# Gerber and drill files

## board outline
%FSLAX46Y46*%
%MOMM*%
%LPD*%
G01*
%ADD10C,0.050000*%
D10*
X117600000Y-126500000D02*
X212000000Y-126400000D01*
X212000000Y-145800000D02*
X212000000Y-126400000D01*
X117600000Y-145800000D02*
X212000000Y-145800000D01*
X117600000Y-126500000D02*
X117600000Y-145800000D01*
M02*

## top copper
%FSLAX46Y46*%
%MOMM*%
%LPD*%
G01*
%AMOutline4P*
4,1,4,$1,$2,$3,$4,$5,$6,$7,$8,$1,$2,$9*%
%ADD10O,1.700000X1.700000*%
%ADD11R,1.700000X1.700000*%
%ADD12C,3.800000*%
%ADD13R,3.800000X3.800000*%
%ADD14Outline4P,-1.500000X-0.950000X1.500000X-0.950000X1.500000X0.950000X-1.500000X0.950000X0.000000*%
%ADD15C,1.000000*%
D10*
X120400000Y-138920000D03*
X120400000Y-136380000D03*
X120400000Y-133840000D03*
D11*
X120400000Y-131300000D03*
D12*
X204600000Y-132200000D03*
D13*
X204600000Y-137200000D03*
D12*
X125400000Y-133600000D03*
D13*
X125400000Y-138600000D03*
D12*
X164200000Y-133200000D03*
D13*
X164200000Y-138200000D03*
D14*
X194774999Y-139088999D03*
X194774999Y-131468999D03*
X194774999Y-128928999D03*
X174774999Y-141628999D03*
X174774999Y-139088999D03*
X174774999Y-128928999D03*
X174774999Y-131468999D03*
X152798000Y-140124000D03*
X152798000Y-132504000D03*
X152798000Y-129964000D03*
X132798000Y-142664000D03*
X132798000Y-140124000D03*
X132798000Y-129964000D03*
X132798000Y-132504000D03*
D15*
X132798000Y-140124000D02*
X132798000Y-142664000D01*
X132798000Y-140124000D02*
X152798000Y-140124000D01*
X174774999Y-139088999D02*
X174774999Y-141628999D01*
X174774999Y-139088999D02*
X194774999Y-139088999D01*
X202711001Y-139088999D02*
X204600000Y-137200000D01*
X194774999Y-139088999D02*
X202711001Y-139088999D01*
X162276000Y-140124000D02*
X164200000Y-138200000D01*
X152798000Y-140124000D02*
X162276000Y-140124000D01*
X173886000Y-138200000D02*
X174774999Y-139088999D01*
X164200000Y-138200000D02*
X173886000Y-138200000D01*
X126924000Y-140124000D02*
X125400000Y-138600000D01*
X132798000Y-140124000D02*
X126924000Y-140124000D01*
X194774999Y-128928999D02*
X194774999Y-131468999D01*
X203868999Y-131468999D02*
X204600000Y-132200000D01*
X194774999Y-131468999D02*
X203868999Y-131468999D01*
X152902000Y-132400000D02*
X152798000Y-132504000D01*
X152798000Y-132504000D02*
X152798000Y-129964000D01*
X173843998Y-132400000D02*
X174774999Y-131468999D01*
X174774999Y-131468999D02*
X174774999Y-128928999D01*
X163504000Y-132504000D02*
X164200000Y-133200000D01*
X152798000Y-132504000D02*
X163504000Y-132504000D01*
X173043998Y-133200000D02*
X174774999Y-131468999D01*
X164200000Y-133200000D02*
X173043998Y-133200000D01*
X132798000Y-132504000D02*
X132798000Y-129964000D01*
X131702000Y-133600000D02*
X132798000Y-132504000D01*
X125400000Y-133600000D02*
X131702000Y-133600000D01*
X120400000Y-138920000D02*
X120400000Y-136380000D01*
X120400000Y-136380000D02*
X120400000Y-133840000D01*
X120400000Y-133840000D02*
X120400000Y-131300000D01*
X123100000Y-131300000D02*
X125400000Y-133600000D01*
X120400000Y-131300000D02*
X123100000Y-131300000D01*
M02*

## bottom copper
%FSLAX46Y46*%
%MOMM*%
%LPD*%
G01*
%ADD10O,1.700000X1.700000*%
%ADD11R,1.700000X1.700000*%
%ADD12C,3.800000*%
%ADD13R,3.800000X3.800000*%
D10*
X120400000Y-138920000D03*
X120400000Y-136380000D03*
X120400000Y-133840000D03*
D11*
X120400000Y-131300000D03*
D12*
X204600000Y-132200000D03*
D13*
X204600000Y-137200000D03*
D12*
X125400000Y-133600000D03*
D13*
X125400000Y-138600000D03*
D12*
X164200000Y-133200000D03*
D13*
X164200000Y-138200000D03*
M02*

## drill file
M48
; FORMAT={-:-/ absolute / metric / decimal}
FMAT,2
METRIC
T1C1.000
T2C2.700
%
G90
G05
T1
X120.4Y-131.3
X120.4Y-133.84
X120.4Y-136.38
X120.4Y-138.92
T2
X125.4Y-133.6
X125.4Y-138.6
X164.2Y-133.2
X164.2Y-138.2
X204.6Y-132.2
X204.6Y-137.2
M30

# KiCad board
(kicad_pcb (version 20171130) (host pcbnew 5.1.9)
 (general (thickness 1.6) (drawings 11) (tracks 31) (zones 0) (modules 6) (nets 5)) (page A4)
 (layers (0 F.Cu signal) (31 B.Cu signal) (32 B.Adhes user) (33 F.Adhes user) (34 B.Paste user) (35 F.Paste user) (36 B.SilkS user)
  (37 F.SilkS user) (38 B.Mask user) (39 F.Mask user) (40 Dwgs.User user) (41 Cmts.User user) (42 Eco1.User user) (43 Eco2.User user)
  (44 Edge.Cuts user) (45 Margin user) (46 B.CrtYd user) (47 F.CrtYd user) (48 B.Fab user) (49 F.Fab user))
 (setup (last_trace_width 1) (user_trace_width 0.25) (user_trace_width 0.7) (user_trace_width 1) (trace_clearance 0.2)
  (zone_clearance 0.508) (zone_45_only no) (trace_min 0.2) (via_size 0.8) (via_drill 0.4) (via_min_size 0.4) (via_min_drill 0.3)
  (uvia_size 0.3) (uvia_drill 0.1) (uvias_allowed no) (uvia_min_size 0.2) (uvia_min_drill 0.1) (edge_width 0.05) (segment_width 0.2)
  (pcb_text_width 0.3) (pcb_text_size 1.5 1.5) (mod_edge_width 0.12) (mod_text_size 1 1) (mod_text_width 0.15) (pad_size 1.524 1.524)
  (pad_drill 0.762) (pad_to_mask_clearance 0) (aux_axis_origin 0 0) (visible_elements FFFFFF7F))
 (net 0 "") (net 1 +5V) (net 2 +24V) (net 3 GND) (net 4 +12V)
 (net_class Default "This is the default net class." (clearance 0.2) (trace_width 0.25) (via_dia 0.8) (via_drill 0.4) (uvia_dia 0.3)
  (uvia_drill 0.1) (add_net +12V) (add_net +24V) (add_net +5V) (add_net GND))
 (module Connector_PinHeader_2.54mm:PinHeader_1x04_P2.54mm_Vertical (layer F.Cu) (at 120.4 131.3)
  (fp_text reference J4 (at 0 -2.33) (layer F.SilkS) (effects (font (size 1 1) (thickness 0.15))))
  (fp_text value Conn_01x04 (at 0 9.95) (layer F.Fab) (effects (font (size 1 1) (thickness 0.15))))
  (pad 4 thru_hole oval (at 0 7.62) (size 1.7 1.7) (drill 1) (layers *.Cu *.Mask) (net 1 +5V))
  (pad 3 thru_hole oval (at 0 5.08) (size 1.7 1.7) (drill 1) (layers *.Cu *.Mask) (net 1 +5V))
  (pad 2 thru_hole oval (at 0 2.54) (size 1.7 1.7) (drill 1) (layers *.Cu *.Mask) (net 1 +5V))
  (pad 1 thru_hole rect (at 0 0) (size 1.7 1.7) (drill 1) (layers *.Cu *.Mask) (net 1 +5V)))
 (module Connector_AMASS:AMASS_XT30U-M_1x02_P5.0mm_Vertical (layer F.Cu) (at 204.6 137.2 90)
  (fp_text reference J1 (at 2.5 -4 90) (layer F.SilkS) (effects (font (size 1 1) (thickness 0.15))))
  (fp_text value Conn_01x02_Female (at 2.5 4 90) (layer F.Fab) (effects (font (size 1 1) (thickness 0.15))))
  (pad 2 thru_hole circle (at 5 0 90) (size 3.8 3.8) (drill 2.7) (layers *.Cu *.Mask) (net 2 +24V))
  (pad 1 thru_hole rect (at 0 0 90) (size 3.8 3.8) (drill 2.7) (layers *.Cu *.Mask) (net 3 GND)))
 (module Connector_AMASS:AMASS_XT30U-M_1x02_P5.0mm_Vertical (layer F.Cu) (at 125.4 138.6 90)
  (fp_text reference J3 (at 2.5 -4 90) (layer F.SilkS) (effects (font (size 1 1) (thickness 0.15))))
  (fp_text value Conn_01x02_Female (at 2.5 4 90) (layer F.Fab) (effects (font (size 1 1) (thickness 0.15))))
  (pad 2 thru_hole circle (at 5 0 90) (size 3.8 3.8) (drill 2.7) (layers *.Cu *.Mask) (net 1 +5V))
  (pad 1 thru_hole rect (at 0 0 90) (size 3.8 3.8) (drill 2.7) (layers *.Cu *.Mask) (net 3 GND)))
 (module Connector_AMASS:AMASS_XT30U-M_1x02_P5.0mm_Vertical (layer F.Cu) (at 164.2 138.2 90)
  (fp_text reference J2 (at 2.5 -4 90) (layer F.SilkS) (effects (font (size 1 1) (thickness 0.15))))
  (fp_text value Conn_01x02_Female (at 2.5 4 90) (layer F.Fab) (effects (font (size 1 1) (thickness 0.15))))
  (pad 2 thru_hole circle (at 5 0 90) (size 3.8 3.8) (drill 2.7) (layers *.Cu *.Mask) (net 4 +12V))
  (pad 1 thru_hole rect (at 0 0 90) (size 3.8 3.8) (drill 2.7) (layers *.Cu *.Mask) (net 3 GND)))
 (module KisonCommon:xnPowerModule (layer F.Cu) (at 178.076999 124.864999)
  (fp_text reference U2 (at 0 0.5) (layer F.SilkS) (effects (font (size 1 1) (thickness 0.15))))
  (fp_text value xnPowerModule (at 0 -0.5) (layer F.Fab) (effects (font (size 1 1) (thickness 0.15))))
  (pad 4 smd trapezoid (at 16.698 14.224) (size 3 1.9) (layers F.Cu F.Paste F.Mask) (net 3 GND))
  (pad 3 smd trapezoid (at 16.698 6.604) (size 3 1.9) (layers F.Cu F.Paste F.Mask) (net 2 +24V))
  (pad 3 smd trapezoid (at 16.698 4.064) (size 3 1.9) (layers F.Cu F.Paste F.Mask) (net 2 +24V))
  (pad 2 smd trapezoid (at -3.302 16.764) (size 3 1.9) (layers F.Cu F.Paste F.Mask) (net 3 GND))
  (pad 2 smd trapezoid (at -3.302 14.224) (size 3 1.9) (layers F.Cu F.Paste F.Mask) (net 3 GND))
  (pad 1 smd trapezoid (at -3.302 4.064) (size 3 1.9) (layers F.Cu F.Paste F.Mask) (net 4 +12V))
  (pad 1 smd trapezoid (at -3.302 6.604) (size 3 1.9) (layers F.Cu F.Paste F.Mask) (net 4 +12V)))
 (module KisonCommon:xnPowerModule (layer F.Cu) (at 136.1 125.9)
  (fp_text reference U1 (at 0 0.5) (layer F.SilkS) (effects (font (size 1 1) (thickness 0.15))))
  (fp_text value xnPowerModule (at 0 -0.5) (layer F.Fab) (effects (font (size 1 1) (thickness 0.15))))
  (pad 4 smd trapezoid (at 16.698 14.224) (size 3 1.9) (layers F.Cu F.Paste F.Mask) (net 3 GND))
  (pad 3 smd trapezoid (at 16.698 6.604) (size 3 1.9) (layers F.Cu F.Paste F.Mask) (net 4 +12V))
  (pad 3 smd trapezoid (at 16.698 4.064) (size 3 1.9) (layers F.Cu F.Paste F.Mask) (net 4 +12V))
  (pad 2 smd trapezoid (at -3.302 16.764) (size 3 1.9) (layers F.Cu F.Paste F.Mask) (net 3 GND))
  (pad 2 smd trapezoid (at -3.302 14.224) (size 3 1.9) (layers F.Cu F.Paste F.Mask) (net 3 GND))
  (pad 1 smd trapezoid (at -3.302 4.064) (size 3 1.9) (layers F.Cu F.Paste F.Mask) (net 1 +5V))
  (pad 1 smd trapezoid (at -3.302 6.604) (size 3 1.9) (layers F.Cu F.Paste F.Mask) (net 1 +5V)))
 (gr_line (start 117.6 126.5) (end 212 126.4) (layer Edge.Cuts) (width 0.05))
 (gr_line (start 212 145.8) (end 212 126.4) (layer Edge.Cuts) (width 0.05))
 (gr_line (start 117.6 145.8) (end 212 145.8) (layer Edge.Cuts) (width 0.05))
 (gr_line (start 117.6 126.5) (end 117.6 145.8) (layer Edge.Cuts) (width 0.05))
 (segment (start 132.798 140.124) (end 132.798 142.664) (width 1) (layer F.Cu) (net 3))
 (segment (start 132.798 140.124) (end 152.798 140.124) (width 1) (layer F.Cu) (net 3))
 (segment (start 174.774999 139.088999) (end 174.774999 141.628999) (width 1) (layer F.Cu) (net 3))
 (segment (start 174.774999 139.088999) (end 194.774999 139.088999) (width 1) (layer F.Cu) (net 3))
 (segment (start 202.711001 139.088999) (end 204.6 137.2) (width 1) (layer F.Cu) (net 3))
 (segment (start 194.774999 139.088999) (end 202.711001 139.088999) (width 1) (layer F.Cu) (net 3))
 (segment (start 162.276 140.124) (end 164.2 138.2) (width 1) (layer F.Cu) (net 3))
 (segment (start 152.798 140.124) (end 162.276 140.124) (width 1) (layer F.Cu) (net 3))
 (segment (start 173.886 138.2) (end 174.774999 139.088999) (width 1) (layer F.Cu) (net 3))
 (segment (start 164.2 138.2) (end 173.886 138.2) (width 1) (layer F.Cu) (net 3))
 (segment (start 126.924 140.124) (end 125.4 138.6) (width 1) (layer F.Cu) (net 3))
 (segment (start 132.798 140.124) (end 126.924 140.124) (width 1) (layer F.Cu) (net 3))
 (segment (start 194.774999 128.928999) (end 194.774999 131.468999) (width 1) (layer F.Cu) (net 2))
 (segment (start 203.868999 131.468999) (end 204.6 132.2) (width 1) (layer F.Cu) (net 2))
 (segment (start 194.774999 131.468999) (end 203.868999 131.468999) (width 1) (layer F.Cu) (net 2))
 (segment (start 152.902 132.4) (end 152.798 132.504) (width 1) (layer F.Cu) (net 4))
 (segment (start 152.798 132.504) (end 152.798 129.964) (width 1) (layer F.Cu) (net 4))
 (segment (start 173.843998 132.4) (end 174.774999 131.468999) (width 1) (layer F.Cu) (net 4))
 (segment (start 174.774999 131.468999) (end 174.774999 128.928999) (width 1) (layer F.Cu) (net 4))
 (segment (start 163.504 132.504) (end 164.2 133.2) (width 1) (layer F.Cu) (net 4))
 (segment (start 152.798 132.504) (end 163.504 132.504) (width 1) (layer F.Cu) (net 4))
 (segment (start 173.043998 133.2) (end 174.774999 131.468999) (width 1) (layer F.Cu) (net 4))
 (segment (start 164.2 133.2) (end 173.043998 133.2) (width 1) (layer F.Cu) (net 4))
 (segment (start 132.798 132.504) (end 132.798 129.964) (width 1) (layer F.Cu) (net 1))
 (segment (start 131.702 133.6) (end 132.798 132.504) (width 1) (layer F.Cu) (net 1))
 (segment (start 125.4 133.6) (end 131.702 133.6) (width 1) (layer F.Cu) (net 1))
 (segment (start 120.4 138.92) (end 120.4 136.38) (width 1) (layer F.Cu) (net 1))
 (segment (start 120.4 136.38) (end 120.4 133.84) (width 1) (layer F.Cu) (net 1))
 (segment (start 120.4 133.84) (end 120.4 131.3) (width 1) (layer F.Cu) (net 1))
 (segment (start 123.1 131.3) (end 125.4 133.6) (width 1) (layer F.Cu) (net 1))
 (segment (start 120.4 131.3) (end 123.1 131.3) (width 1) (layer F.Cu) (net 1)))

